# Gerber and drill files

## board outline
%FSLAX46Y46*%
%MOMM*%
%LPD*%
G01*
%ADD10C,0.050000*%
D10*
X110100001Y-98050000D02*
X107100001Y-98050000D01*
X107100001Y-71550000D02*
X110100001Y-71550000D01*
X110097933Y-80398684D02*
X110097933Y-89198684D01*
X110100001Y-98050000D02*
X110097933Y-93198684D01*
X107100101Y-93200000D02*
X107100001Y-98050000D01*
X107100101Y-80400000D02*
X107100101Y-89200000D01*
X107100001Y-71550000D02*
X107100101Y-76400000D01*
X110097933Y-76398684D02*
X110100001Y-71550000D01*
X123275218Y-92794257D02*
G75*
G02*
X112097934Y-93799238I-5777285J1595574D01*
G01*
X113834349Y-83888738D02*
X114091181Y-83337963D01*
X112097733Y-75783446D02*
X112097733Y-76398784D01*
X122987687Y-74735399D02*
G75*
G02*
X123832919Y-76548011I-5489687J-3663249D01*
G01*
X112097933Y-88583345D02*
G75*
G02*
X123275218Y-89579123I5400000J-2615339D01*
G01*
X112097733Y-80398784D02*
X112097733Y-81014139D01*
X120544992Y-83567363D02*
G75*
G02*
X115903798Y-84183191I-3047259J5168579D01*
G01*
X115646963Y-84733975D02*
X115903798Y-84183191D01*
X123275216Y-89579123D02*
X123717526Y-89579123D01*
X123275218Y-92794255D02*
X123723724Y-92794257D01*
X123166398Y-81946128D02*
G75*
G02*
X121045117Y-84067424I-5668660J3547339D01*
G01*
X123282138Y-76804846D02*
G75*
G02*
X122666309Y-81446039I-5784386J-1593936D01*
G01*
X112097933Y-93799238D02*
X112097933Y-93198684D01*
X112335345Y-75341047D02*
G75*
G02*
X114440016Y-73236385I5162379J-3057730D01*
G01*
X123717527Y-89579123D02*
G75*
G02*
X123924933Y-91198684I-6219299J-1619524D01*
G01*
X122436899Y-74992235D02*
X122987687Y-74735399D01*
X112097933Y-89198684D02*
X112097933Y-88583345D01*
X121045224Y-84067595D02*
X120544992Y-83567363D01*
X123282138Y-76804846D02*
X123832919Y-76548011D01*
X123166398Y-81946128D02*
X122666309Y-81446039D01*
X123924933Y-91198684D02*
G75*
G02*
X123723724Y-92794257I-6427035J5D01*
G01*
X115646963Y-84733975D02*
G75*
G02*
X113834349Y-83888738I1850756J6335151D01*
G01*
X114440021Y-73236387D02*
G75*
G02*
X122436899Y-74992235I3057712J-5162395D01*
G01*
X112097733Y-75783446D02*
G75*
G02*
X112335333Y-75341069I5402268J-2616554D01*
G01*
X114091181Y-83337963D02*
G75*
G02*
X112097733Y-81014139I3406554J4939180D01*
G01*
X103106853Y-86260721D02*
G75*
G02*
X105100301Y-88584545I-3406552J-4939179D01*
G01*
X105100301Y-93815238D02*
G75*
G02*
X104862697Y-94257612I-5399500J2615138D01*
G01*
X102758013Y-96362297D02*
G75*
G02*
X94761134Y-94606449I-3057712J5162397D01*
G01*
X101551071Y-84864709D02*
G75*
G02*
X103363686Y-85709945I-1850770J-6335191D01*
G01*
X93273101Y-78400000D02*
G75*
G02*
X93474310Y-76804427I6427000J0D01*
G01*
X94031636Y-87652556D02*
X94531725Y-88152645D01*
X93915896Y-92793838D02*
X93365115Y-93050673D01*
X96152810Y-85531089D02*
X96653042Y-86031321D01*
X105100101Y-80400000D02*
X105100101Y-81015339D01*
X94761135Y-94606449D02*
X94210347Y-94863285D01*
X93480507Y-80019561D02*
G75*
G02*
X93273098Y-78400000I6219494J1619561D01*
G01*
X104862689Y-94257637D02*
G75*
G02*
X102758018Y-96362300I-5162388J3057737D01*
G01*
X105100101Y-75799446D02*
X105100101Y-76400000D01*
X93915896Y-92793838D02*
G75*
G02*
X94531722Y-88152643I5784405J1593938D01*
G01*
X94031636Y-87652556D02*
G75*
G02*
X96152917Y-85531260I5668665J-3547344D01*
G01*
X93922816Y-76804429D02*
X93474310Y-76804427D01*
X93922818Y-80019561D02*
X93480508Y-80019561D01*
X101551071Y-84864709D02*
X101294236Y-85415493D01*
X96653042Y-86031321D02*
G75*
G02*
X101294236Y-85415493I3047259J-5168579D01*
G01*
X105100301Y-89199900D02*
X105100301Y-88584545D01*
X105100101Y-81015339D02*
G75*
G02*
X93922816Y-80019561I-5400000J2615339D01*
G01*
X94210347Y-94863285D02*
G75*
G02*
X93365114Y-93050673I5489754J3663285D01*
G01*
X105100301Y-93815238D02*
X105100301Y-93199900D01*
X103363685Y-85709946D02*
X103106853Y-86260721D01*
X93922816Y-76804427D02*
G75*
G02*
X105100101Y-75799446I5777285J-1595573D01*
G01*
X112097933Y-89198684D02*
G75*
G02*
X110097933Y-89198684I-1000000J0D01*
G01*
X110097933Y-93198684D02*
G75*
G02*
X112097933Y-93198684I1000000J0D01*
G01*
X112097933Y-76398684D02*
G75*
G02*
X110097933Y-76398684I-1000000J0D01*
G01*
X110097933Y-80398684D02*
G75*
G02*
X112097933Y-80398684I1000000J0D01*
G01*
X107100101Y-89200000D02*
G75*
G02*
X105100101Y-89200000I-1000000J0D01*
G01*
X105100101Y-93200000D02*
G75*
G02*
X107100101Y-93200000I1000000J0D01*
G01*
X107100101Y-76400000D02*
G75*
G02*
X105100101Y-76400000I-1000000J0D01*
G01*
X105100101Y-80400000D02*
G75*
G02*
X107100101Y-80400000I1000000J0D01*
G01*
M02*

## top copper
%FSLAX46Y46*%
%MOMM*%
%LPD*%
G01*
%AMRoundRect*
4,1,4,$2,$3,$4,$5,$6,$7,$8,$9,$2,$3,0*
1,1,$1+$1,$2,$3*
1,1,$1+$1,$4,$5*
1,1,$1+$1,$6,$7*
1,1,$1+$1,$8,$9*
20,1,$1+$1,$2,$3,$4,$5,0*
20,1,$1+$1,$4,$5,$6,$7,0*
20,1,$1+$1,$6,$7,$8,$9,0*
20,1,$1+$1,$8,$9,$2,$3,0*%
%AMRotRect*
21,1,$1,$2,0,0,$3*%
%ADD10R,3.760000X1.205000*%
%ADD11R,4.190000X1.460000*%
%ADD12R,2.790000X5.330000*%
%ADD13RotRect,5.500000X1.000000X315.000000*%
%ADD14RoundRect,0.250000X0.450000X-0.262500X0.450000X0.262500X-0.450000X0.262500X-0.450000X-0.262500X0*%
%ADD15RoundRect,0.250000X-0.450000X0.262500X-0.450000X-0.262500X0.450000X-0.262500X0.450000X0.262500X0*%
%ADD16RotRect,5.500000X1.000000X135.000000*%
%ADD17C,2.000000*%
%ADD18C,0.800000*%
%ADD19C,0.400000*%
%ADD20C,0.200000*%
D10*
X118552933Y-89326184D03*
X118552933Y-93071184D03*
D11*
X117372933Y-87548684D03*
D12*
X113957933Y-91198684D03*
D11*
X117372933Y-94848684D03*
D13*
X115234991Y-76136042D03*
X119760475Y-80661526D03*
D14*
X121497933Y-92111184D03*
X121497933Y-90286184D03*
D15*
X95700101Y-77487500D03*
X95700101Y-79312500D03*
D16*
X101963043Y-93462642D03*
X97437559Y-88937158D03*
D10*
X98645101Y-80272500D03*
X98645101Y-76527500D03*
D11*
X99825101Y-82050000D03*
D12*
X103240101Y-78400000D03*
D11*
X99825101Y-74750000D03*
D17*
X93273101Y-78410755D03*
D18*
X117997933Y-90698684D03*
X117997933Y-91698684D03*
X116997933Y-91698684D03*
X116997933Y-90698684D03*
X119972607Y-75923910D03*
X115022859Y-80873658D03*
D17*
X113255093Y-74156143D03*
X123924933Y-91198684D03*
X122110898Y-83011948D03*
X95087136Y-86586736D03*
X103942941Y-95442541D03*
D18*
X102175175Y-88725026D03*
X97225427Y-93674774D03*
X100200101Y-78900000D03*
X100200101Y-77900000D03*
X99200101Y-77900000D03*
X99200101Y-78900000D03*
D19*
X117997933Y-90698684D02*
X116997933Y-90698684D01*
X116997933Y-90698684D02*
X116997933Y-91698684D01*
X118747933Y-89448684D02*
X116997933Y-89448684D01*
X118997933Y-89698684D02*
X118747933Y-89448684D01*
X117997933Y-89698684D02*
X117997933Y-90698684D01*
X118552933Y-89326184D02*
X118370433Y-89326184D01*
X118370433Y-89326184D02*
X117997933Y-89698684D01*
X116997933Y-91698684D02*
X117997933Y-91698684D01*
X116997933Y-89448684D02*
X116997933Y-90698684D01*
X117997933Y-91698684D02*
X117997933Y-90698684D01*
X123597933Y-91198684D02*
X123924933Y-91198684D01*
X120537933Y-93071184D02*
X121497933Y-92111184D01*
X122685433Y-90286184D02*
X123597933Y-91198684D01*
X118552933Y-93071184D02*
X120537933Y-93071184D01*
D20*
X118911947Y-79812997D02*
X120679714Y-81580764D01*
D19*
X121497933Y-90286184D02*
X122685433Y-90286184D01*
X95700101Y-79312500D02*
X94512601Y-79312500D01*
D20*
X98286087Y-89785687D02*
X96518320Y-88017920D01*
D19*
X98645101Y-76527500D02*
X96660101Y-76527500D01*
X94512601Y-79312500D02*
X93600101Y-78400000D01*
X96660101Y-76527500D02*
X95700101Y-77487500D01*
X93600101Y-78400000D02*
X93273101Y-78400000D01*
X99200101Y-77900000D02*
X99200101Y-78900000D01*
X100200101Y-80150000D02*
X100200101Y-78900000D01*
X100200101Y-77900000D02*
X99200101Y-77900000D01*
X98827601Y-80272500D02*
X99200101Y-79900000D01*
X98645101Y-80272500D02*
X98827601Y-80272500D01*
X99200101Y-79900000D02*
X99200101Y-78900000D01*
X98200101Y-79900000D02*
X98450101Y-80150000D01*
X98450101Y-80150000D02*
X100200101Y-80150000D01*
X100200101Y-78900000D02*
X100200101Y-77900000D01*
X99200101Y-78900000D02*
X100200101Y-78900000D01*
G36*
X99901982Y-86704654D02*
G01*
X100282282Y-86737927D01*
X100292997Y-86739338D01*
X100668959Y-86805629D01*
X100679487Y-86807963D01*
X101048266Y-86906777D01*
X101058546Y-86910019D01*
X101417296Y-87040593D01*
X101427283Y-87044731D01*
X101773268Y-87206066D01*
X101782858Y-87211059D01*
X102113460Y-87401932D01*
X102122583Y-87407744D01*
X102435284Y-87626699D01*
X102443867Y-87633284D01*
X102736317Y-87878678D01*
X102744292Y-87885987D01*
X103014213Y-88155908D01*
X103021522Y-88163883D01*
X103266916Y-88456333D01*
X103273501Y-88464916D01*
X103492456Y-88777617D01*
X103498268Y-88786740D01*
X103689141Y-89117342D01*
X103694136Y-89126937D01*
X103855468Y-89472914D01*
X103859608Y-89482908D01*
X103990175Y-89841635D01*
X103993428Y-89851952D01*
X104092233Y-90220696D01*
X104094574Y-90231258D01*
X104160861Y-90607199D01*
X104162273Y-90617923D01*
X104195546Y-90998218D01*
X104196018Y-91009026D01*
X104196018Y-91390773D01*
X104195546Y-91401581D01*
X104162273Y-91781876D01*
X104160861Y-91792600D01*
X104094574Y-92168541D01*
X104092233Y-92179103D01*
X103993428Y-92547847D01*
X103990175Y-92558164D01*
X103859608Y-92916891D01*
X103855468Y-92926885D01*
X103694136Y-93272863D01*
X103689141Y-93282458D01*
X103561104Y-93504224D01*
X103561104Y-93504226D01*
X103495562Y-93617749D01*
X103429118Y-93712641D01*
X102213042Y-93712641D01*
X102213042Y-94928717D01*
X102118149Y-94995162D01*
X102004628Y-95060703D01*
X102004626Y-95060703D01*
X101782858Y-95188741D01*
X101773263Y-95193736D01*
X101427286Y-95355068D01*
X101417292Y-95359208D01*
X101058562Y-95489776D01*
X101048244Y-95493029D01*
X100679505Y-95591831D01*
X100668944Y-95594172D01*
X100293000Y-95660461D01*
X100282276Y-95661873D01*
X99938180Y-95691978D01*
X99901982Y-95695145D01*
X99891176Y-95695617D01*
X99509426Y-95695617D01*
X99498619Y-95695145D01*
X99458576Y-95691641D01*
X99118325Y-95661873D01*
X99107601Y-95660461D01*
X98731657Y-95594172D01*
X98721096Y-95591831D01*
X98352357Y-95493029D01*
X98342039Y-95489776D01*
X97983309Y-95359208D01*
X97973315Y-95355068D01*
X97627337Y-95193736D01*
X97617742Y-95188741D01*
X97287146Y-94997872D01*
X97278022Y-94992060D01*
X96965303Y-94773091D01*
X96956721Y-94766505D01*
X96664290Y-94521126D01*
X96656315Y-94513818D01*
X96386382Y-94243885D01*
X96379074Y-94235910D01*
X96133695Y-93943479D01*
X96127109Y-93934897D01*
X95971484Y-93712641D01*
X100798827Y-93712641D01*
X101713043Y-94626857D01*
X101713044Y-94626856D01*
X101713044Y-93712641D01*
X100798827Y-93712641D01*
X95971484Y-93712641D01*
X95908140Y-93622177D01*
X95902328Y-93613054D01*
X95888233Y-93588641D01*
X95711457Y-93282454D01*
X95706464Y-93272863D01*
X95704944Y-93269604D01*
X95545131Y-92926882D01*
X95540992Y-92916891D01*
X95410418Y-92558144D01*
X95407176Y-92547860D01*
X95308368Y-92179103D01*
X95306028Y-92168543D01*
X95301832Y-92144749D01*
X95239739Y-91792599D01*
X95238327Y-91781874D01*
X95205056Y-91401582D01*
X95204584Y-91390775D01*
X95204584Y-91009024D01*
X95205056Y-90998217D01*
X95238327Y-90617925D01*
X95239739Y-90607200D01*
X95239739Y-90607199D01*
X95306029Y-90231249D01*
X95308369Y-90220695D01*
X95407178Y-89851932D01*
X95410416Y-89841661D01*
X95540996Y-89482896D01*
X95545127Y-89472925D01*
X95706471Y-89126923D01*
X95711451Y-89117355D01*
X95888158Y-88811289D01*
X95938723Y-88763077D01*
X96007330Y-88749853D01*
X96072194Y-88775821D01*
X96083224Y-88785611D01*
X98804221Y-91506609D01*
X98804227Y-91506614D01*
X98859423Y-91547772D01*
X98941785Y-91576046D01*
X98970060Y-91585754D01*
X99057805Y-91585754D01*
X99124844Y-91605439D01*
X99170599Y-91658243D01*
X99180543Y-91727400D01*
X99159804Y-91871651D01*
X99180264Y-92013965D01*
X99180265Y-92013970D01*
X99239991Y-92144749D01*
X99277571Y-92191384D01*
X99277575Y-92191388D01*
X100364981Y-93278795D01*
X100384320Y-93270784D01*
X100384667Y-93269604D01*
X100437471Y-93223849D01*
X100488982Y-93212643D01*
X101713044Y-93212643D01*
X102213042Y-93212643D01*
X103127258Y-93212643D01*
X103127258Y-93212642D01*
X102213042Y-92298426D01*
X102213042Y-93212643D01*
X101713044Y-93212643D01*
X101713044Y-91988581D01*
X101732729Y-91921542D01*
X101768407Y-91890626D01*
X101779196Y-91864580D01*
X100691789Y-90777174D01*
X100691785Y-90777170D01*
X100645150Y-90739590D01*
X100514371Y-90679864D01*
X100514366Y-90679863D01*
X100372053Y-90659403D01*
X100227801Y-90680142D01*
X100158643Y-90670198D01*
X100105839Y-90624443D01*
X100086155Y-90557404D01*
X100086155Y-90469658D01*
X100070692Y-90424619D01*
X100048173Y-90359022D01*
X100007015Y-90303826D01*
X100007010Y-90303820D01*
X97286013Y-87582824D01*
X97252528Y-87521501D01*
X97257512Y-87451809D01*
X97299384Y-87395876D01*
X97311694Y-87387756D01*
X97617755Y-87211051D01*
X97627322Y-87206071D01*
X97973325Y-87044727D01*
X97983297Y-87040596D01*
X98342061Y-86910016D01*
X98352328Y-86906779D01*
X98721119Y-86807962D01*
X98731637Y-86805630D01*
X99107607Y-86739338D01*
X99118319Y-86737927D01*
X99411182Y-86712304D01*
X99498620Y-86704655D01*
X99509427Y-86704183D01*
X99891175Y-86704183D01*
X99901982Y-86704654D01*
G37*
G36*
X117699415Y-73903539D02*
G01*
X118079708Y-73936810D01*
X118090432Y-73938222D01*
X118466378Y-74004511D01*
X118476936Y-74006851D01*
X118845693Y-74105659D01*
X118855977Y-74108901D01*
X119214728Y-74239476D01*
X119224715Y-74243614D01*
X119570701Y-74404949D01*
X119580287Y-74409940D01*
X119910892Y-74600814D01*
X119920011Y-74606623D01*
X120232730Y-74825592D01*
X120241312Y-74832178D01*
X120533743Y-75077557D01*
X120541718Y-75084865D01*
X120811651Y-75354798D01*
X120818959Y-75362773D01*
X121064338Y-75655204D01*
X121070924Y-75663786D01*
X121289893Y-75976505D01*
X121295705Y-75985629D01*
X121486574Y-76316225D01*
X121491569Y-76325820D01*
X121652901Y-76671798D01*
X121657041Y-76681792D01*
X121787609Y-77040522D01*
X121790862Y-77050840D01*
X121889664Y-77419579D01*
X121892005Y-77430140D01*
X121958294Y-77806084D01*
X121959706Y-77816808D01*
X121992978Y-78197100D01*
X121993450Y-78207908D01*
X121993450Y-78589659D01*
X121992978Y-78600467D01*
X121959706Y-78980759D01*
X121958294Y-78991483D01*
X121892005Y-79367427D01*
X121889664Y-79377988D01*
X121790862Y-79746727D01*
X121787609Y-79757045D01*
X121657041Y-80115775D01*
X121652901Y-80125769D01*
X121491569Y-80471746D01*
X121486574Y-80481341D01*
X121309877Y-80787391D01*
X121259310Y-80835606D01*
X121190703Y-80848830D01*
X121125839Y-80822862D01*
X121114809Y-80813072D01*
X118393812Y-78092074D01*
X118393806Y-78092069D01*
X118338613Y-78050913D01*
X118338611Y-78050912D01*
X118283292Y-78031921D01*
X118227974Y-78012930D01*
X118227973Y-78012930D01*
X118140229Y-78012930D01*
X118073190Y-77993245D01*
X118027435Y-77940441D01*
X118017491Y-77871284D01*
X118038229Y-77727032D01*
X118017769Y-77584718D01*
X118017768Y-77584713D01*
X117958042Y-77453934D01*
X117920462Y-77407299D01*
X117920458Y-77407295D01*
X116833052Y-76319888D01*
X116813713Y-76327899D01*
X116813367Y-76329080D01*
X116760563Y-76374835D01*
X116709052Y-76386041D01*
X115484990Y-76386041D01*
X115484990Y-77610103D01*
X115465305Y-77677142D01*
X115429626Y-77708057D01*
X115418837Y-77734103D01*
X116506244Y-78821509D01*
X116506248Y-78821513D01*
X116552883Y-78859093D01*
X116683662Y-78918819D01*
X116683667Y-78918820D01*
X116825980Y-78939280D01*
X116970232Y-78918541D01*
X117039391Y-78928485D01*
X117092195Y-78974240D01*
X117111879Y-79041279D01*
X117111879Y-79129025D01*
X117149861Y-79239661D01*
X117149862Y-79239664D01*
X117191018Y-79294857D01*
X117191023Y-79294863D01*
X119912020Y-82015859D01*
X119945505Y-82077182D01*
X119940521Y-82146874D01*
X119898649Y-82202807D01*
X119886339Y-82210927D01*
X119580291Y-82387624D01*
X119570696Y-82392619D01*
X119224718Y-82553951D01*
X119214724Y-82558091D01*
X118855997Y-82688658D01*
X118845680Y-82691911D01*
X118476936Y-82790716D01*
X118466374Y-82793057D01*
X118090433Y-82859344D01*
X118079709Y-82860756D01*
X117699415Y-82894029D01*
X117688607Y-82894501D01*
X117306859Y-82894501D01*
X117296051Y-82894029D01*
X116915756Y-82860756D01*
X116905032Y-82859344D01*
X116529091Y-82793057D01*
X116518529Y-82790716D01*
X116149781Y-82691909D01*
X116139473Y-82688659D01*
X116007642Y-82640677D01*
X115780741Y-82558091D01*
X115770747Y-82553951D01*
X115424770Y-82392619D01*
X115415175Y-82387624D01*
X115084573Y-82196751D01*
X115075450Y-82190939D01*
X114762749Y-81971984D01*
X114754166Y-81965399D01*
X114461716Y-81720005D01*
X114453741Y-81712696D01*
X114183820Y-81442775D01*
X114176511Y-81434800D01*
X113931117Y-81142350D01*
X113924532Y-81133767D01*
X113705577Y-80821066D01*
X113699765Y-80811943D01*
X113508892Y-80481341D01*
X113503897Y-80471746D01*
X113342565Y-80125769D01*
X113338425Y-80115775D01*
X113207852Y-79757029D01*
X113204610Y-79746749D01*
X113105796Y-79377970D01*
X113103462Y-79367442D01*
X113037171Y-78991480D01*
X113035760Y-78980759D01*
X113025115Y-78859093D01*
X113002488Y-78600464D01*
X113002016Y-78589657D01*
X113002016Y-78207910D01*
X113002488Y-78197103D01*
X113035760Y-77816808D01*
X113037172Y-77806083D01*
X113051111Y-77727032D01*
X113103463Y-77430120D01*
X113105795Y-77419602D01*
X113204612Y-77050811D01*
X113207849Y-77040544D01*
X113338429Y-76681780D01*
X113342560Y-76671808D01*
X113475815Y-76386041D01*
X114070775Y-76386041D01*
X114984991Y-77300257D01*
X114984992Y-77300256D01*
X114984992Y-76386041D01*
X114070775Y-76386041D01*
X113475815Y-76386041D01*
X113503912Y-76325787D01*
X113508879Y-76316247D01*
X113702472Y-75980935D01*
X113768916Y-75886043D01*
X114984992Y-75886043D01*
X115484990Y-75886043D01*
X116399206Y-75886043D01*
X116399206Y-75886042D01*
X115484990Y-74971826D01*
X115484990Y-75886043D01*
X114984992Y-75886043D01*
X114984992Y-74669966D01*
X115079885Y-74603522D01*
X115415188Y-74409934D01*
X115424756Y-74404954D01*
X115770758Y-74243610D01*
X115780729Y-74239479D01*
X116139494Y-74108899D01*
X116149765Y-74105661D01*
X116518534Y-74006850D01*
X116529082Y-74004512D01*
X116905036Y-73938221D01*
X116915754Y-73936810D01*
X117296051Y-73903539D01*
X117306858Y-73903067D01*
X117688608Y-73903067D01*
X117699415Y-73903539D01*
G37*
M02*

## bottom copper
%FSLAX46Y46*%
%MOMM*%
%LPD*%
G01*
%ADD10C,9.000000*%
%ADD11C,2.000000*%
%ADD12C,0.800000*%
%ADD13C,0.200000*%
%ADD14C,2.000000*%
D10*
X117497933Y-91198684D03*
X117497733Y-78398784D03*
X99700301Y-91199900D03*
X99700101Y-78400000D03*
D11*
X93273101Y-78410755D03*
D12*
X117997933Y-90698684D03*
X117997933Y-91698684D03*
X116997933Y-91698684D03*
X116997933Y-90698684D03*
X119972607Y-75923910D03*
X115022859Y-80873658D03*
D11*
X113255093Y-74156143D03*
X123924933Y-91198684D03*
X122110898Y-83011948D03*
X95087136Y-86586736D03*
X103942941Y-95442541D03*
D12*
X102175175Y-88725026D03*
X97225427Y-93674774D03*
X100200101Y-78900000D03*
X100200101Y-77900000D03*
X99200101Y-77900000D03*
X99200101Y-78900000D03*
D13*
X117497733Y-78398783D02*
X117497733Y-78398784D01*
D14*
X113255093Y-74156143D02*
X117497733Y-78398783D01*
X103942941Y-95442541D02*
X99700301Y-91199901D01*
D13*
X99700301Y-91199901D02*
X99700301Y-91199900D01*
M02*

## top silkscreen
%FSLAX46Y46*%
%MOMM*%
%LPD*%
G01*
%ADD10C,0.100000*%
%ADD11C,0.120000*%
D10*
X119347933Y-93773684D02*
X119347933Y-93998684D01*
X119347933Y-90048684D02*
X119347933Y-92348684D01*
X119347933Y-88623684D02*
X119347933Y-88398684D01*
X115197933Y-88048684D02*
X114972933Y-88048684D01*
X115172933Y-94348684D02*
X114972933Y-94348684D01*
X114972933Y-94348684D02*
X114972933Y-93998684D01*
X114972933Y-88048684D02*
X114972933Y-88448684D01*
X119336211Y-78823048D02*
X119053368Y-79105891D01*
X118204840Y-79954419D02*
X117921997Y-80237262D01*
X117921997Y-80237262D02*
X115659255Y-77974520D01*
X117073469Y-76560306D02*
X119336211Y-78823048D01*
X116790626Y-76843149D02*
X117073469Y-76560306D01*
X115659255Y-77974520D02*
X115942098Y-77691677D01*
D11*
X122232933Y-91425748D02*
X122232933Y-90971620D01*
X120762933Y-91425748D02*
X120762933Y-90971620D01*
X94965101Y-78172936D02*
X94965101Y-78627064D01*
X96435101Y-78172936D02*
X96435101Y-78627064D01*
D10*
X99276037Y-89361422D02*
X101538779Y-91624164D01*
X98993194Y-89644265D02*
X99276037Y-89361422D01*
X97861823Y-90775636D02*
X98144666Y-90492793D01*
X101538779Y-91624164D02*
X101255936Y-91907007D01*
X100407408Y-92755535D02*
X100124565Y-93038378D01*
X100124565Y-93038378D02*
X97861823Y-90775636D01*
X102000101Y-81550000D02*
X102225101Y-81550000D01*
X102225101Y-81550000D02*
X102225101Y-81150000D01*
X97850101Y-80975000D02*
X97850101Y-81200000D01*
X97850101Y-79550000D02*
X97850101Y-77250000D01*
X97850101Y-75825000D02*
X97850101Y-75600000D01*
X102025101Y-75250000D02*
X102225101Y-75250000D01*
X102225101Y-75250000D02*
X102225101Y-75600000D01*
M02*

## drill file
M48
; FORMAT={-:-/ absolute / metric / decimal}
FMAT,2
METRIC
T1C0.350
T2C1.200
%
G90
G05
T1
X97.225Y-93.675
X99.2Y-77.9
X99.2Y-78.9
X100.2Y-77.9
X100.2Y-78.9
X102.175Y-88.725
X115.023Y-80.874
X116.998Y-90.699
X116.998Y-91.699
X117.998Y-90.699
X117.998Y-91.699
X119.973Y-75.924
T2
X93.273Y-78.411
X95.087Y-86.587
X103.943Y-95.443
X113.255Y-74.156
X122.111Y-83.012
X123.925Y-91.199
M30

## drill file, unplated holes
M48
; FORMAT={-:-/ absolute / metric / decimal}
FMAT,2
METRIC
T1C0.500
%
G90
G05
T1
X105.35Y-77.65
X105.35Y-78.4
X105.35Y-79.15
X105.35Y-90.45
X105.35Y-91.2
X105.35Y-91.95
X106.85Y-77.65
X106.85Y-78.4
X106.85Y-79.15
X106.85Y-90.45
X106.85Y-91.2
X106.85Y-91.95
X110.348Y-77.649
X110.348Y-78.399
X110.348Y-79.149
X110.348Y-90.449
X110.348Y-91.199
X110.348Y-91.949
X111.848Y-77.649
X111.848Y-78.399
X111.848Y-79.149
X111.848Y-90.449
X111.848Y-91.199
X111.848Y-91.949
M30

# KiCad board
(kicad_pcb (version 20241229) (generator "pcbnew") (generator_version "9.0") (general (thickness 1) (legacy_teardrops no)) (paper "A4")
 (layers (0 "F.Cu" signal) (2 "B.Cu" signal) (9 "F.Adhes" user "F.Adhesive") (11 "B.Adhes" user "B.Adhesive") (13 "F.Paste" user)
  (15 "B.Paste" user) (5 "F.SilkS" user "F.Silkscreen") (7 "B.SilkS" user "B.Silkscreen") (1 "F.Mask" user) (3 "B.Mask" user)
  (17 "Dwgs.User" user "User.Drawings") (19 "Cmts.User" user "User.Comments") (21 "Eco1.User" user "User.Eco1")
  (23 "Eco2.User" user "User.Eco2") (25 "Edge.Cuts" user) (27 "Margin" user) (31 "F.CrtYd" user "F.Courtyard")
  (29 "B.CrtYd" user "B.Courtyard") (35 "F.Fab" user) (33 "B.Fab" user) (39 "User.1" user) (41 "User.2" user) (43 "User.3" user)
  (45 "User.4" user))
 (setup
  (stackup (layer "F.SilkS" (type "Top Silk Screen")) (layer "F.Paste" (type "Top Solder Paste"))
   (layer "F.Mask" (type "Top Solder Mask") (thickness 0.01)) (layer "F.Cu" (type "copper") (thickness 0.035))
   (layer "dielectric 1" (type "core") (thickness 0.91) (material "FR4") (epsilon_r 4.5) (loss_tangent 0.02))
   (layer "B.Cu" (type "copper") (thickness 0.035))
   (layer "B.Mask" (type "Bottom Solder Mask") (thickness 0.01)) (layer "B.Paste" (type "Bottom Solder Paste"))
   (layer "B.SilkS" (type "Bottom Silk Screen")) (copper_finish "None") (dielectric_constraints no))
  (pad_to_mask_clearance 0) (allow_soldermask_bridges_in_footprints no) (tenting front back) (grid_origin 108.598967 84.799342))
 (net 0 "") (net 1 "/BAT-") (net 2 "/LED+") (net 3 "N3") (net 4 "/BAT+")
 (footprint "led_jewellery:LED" (layer "F.Cu") (at 99.700301 91.1999 135)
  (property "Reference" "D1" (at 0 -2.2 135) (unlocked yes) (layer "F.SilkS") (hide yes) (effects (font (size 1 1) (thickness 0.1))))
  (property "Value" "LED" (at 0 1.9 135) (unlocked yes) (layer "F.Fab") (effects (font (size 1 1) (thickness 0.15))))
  (fp_line (start 1.6 -1) (end 1.6 -0.6) (stroke (width 0.1) (type default)) (layer "F.SilkS"))
  (fp_line (start 1.6 0.6) (end 1.6 1) (stroke (width 0.1) (type default)) (layer "F.SilkS"))
  (fp_line (start 1.6 1) (end -1.6 1) (stroke (width 0.1) (type default)) (layer "F.SilkS"))
  (fp_line (start -1.6 -1) (end 1.6 -1) (stroke (width 0.1) (type default)) (layer "F.SilkS"))
  (fp_line (start -1.6 -0.6) (end -1.6 -1) (stroke (width 0.1) (type default)) (layer "F.SilkS"))
  (fp_line (start -1.6 1) (end -1.6 0.6) (stroke (width 0.1) (type default)) (layer "F.SilkS"))
  (pad "1" smd rect (at -3.2 0 135) (size 5.5 1) (layers "F.Cu" "F.Mask") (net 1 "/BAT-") (thermal_bridge_angle 45))
  (pad "2" smd rect (at 3.2 0 135) (size 5.5 1) (layers "F.Cu" "F.Mask") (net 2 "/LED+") (thermal_bridge_angle 45)))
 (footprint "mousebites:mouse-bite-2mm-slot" (layer "F.Cu") (at 106.100101 78.4 90)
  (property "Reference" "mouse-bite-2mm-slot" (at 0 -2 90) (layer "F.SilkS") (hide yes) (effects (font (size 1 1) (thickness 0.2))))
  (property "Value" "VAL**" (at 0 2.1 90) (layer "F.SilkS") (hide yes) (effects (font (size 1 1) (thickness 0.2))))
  (fp_arc (start -2 -1) (mid -1 0) (end -2 1) (stroke (width 0.05) (type solid)) (layer "Edge.Cuts"))
  (fp_arc (start 2 1) (mid 1 0) (end 2 -1) (stroke (width 0.05) (type solid)) (layer "Edge.Cuts"))
  (pad "" np_thru_hole circle (at -0.75 -0.75 90) (size 0.5 0.5) (drill 0.5) (layers "*.Cu" "*.Mask"))
  (pad "" np_thru_hole circle (at -0.75 0.75 90) (size 0.5 0.5) (drill 0.5) (layers "*.Cu" "*.Mask"))
  (pad "" np_thru_hole circle (at 0 -0.75 90) (size 0.5 0.5) (drill 0.5) (layers "*.Cu" "*.Mask"))
  (pad "" np_thru_hole circle (at 0 0.75 90) (size 0.5 0.5) (drill 0.5) (layers "*.Cu" "*.Mask"))
  (pad "" np_thru_hole circle (at 0.75 -0.75 90) (size 0.5 0.5) (drill 0.5) (layers "*.Cu" "*.Mask"))
  (pad "" np_thru_hole circle (at 0.75 0.75 90) (size 0.5 0.5) (drill 0.5) (layers "*.Cu" "*.Mask")))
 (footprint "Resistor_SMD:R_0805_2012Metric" (layer "F.Cu") (at 95.700101 78.4 -90)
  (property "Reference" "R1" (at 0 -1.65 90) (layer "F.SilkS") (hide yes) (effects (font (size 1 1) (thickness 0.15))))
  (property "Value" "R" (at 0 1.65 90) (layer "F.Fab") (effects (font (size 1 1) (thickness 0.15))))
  (fp_line (start -0.227064 0.735) (end 0.227064 0.735) (stroke (width 0.12) (type solid)) (layer "F.SilkS"))
  (fp_line (start -0.227064 -0.735) (end 0.227064 -0.735) (stroke (width 0.12) (type solid)) (layer "F.SilkS"))
  (pad "1" smd roundrect (at -0.9125 0 270) (size 1.025 1.4) (layers "F.Cu" "F.Mask" "F.Paste") (roundrect_rratio 0.243902) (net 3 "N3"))
  (pad "2" smd roundrect (at 0.9125 0 270) (size 1.025 1.4) (layers "F.Cu" "F.Mask" "F.Paste") (roundrect_rratio 0.243902) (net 2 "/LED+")))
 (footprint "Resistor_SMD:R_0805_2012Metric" (layer "F.Cu") (at 121.497933 91.198684 90)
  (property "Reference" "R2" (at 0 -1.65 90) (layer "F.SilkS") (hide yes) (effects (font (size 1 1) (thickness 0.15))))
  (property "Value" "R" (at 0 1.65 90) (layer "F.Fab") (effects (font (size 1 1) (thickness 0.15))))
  (fp_line (start -0.227064 -0.735) (end 0.227064 -0.735) (stroke (width 0.12) (type solid)) (layer "F.SilkS"))
  (fp_line (start -0.227064 0.735) (end 0.227064 0.735) (stroke (width 0.12) (type solid)) (layer "F.SilkS"))
  (pad "1" smd roundrect (at -0.9125 0 90) (size 1.025 1.4) (layers "F.Cu" "F.Mask" "F.Paste") (roundrect_rratio 0.243902) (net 3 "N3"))
  (pad "2" smd roundrect (at 0.9125 0 90) (size 1.025 1.4) (layers "F.Cu" "F.Mask" "F.Paste") (roundrect_rratio 0.243902) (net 2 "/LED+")))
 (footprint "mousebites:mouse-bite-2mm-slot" (layer "F.Cu") (at 111.097933 78.398684 -90)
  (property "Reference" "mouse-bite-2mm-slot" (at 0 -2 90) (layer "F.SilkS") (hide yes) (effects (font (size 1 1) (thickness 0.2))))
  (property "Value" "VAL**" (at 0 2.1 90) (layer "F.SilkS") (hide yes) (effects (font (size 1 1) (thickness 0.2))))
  (fp_arc (start 2 1) (mid 1 0) (end 2 -1) (stroke (width 0.05) (type solid)) (layer "Edge.Cuts"))
  (fp_arc (start -2 -1) (mid -1 0) (end -2 1) (stroke (width 0.05) (type solid)) (layer "Edge.Cuts"))
  (pad "" np_thru_hole circle (at -0.75 -0.75 270) (size 0.5 0.5) (drill 0.5) (layers "*.Cu" "*.Mask"))
  (pad "" np_thru_hole circle (at -0.75 0.75 270) (size 0.5 0.5) (drill 0.5) (layers "*.Cu" "*.Mask"))
  (pad "" np_thru_hole circle (at 0 -0.75 270) (size 0.5 0.5) (drill 0.5) (layers "*.Cu" "*.Mask"))
  (pad "" np_thru_hole circle (at 0 0.75 270) (size 0.5 0.5) (drill 0.5) (layers "*.Cu" "*.Mask"))
  (pad "" np_thru_hole circle (at 0.75 -0.75 270) (size 0.5 0.5) (drill 0.5) (layers "*.Cu" "*.Mask"))
  (pad "" np_thru_hole circle (at 0.75 0.75 270) (size 0.5 0.5) (drill 0.5) (layers "*.Cu" "*.Mask")))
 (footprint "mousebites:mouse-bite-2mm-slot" (layer "F.Cu") (at 111.097933 91.198684 -90)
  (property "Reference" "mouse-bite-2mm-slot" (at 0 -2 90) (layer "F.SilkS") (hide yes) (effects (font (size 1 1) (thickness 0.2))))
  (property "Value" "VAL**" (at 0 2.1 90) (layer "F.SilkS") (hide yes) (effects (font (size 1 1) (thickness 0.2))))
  (fp_arc (start 2 1) (mid 1 0) (end 2 -1) (stroke (width 0.05) (type solid)) (layer "Edge.Cuts"))
  (fp_arc (start -2 -1) (mid -1 0) (end -2 1) (stroke (width 0.05) (type solid)) (layer "Edge.Cuts"))
  (pad "" np_thru_hole circle (at -0.75 -0.75 270) (size 0.5 0.5) (drill 0.5) (layers "*.Cu" "*.Mask"))
  (pad "" np_thru_hole circle (at -0.75 0.75 270) (size 0.5 0.5) (drill 0.5) (layers "*.Cu" "*.Mask"))
  (pad "" np_thru_hole circle (at 0 -0.75 270) (size 0.5 0.5) (drill 0.5) (layers "*.Cu" "*.Mask"))
  (pad "" np_thru_hole circle (at 0 0.75 270) (size 0.5 0.5) (drill 0.5) (layers "*.Cu" "*.Mask"))
  (pad "" np_thru_hole circle (at 0.75 -0.75 270) (size 0.5 0.5) (drill 0.5) (layers "*.Cu" "*.Mask"))
  (pad "" np_thru_hole circle (at 0.75 0.75 270) (size 0.5 0.5) (drill 0.5) (layers "*.Cu" "*.Mask")))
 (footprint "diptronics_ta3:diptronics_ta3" (layer "F.Cu") (at 102.225101 78.4 90)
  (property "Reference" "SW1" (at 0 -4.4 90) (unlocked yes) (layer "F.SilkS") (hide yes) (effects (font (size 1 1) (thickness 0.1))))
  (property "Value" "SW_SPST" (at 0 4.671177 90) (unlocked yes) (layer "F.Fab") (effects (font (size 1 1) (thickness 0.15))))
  (fp_line (start 2.575 -4.375) (end 2.8 -4.375) (stroke (width 0.1) (type default)) (layer "F.SilkS"))
  (fp_line (start -1.15 -4.375) (end 1.15 -4.375) (stroke (width 0.1) (type default)) (layer "F.SilkS"))
  (fp_line (start -2.575 -4.375) (end -2.8 -4.375) (stroke (width 0.1) (type default)) (layer "F.SilkS"))
  (fp_line (start -3.15 -0.225) (end -3.15 0) (stroke (width 0.1) (type default)) (layer "F.SilkS"))
  (fp_line (start 3.15 -0.2) (end 3.15 0) (stroke (width 0.1) (type default)) (layer "F.SilkS"))
  (fp_line (start 3.15 0) (end 2.8 0) (stroke (width 0.1) (type default)) (layer "F.SilkS"))
  (fp_line (start -3.15 0) (end -2.75 0) (stroke (width 0.1) (type default)) (layer "F.SilkS"))
  (pad "1" smd rect (at -1.8725 -3.58 180) (size 3.76 1.205) (layers "F.Cu" "F.Mask" "F.Paste") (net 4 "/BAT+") (thermal_bridge_angle 45))
  (pad "2" smd rect (at 1.8725 -3.58 180) (size 3.76 1.205) (layers "F.Cu" "F.Mask" "F.Paste") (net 3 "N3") (thermal_bridge_angle 45))
  (pad "MP" smd rect (at -3.65 -2.4 90) (size 1.46 4.19) (layers "F.Cu" "F.Mask" "F.Paste") (thermal_bridge_angle 45))
  (pad "MP" smd rect (at 0 1.015 90) (size 5.33 2.79) (layers "F.Cu" "F.Mask" "F.Paste") (thermal_bridge_angle 45))
  (pad "MP" smd rect (at 3.65 -2.4 90) (size 1.46 4.19) (layers "F.Cu" "F.Mask" "F.Paste") (thermal_bridge_angle 45)))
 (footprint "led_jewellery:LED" (layer "F.Cu") (at 117.497733 78.398784 -45)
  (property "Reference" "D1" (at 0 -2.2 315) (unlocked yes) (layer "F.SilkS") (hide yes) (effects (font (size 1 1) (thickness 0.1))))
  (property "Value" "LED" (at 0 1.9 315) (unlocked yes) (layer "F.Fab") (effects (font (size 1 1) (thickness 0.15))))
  (fp_line (start -1.6 1) (end -1.6 0.6) (stroke (width 0.1) (type default)) (layer "F.SilkS"))
  (fp_line (start -1.6 -0.6) (end -1.6 -1) (stroke (width 0.1) (type default)) (layer "F.SilkS"))
  (fp_line (start -1.6 -1) (end 1.6 -1) (stroke (width 0.1) (type default)) (layer "F.SilkS"))
  (fp_line (start 1.6 1) (end -1.6 1) (stroke (width 0.1) (type default)) (layer "F.SilkS"))
  (fp_line (start 1.6 0.6) (end 1.6 1) (stroke (width 0.1) (type default)) (layer "F.SilkS"))
  (fp_line (start 1.6 -1) (end 1.6 -0.6) (stroke (width 0.1) (type default)) (layer "F.SilkS"))
  (pad "1" smd rect (at -3.2 0 315) (size 5.5 1) (layers "F.Cu" "F.Mask") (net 1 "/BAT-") (thermal_bridge_angle 45))
  (pad "2" smd rect (at 3.2 0 315) (size 5.5 1) (layers "F.Cu" "F.Mask") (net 2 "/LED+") (thermal_bridge_angle 45)))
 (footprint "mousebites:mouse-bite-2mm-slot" (layer "F.Cu") (at 106.100101 91.2 90)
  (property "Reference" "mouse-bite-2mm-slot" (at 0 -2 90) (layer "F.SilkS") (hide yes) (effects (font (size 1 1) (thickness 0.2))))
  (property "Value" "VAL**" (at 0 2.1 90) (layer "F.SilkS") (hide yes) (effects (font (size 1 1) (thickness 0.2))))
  (fp_arc (start -2 -1) (mid -1 0) (end -2 1) (stroke (width 0.05) (type solid)) (layer "Edge.Cuts"))
  (fp_arc (start 2 1) (mid 1 0) (end 2 -1) (stroke (width 0.05) (type solid)) (layer "Edge.Cuts"))
  (pad "" np_thru_hole circle (at -0.75 -0.75 90) (size 0.5 0.5) (drill 0.5) (layers "*.Cu" "*.Mask"))
  (pad "" np_thru_hole circle (at -0.75 0.75 90) (size 0.5 0.5) (drill 0.5) (layers "*.Cu" "*.Mask"))
  (pad "" np_thru_hole circle (at 0 -0.75 90) (size 0.5 0.5) (drill 0.5) (layers "*.Cu" "*.Mask"))
  (pad "" np_thru_hole circle (at 0 0.75 90) (size 0.5 0.5) (drill 0.5) (layers "*.Cu" "*.Mask"))
  (pad "" np_thru_hole circle (at 0.75 -0.75 90) (size 0.5 0.5) (drill 0.5) (layers "*.Cu" "*.Mask"))
  (pad "" np_thru_hole circle (at 0.75 0.75 90) (size 0.5 0.5) (drill 0.5) (layers "*.Cu" "*.Mask")))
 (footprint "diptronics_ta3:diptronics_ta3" (layer "F.Cu") (at 114.972933 91.198684 -90)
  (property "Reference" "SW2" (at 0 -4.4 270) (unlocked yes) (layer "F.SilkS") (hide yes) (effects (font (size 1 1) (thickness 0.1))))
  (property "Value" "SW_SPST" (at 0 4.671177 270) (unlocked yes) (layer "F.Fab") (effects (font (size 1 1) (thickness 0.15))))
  (fp_line (start -3.15 0) (end -2.75 0) (stroke (width 0.1) (type default)) (layer "F.SilkS"))
  (fp_line (start 3.15 0) (end 2.8 0) (stroke (width 0.1) (type default)) (layer "F.SilkS"))
  (fp_line (start 3.15 -0.2) (end 3.15 0) (stroke (width 0.1) (type default)) (layer "F.SilkS"))
  (fp_line (start -3.15 -0.225) (end -3.15 0) (stroke (width 0.1) (type default)) (layer "F.SilkS"))
  (fp_line (start -2.575 -4.375) (end -2.8 -4.375) (stroke (width 0.1) (type default)) (layer "F.SilkS"))
  (fp_line (start -1.15 -4.375) (end 1.15 -4.375) (stroke (width 0.1) (type default)) (layer "F.SilkS"))
  (fp_line (start 2.575 -4.375) (end 2.8 -4.375) (stroke (width 0.1) (type default)) (layer "F.SilkS"))
  (pad "1" smd rect (at -1.8725 -3.58) (size 3.76 1.205) (layers "F.Cu" "F.Mask" "F.Paste") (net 4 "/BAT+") (thermal_bridge_angle 45))
  (pad "2" smd rect (at 1.8725 -3.58) (size 3.76 1.205) (layers "F.Cu" "F.Mask" "F.Paste") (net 3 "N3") (thermal_bridge_angle 45))
  (pad "MP" smd rect (at -3.65 -2.4 270) (size 1.46 4.19) (layers "F.Cu" "F.Mask" "F.Paste") (thermal_bridge_angle 45))
  (pad "MP" smd rect (at 0 1.015 270) (size 5.33 2.79) (layers "F.Cu" "F.Mask" "F.Paste") (thermal_bridge_angle 45))
  (pad "MP" smd rect (at 3.65 -2.4 270) (size 1.46 4.19) (layers "F.Cu" "F.Mask" "F.Paste") (thermal_bridge_angle 45)))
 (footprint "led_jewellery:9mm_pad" (layer "B.Cu") (at 117.497933 91.198684 90)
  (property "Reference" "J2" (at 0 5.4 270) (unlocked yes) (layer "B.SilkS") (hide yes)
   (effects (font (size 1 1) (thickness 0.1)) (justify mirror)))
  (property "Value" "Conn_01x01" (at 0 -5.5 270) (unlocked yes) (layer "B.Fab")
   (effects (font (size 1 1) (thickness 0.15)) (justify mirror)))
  (pad "1" smd circle (at 0 0 90) (size 9 9) (layers "B.Cu" "B.Mask") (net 4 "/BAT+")))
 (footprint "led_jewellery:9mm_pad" (layer "B.Cu") (at 99.700301 91.1999 135)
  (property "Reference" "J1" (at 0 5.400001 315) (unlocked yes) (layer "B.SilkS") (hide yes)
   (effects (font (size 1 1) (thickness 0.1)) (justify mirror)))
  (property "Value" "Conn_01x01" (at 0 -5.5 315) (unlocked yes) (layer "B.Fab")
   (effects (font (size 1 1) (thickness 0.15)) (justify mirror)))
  (pad "1" smd circle (at 0 0 135) (size 9 9) (layers "B.Cu" "B.Mask") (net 1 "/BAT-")))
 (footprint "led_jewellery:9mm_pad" (layer "B.Cu") (at 117.497733 78.398784 -45)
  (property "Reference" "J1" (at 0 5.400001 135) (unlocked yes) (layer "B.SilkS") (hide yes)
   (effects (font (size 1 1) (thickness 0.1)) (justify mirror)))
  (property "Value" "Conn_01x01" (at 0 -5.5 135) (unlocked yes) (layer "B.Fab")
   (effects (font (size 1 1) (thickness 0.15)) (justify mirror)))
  (pad "1" smd circle (at 0 0 315) (size 9 9) (layers "B.Cu" "B.Mask") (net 1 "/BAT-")))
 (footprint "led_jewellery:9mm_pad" (layer "B.Cu") (at 99.700101 78.4 -90)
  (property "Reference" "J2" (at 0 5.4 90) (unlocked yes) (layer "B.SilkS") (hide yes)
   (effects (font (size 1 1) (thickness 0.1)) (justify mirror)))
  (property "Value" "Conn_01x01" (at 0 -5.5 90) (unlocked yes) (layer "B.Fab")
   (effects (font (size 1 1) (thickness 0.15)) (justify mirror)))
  (pad "1" smd circle (at 0 0 270) (size 9 9) (layers "B.Cu" "B.Mask") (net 4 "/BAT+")))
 (gr_arc (start 103.106853 86.260721) (mid 104.254297 87.293341) (end 105.100301 88.584545) (stroke (width 0.05) (type default))
  (layer "Edge.Cuts"))
 (gr_line (start 122.436899 74.992235) (end 122.987687 74.735399) (stroke (width 0.05) (type solid)) (layer "Edge.Cuts"))
 (gr_arc (start 123.166398 81.946128) (mid 122.226249 83.127267) (end 121.045117 84.067424) (stroke (width 0.05) (type default))
  (layer "Edge.Cuts"))
 (gr_line (start 123.275216 89.579123) (end 123.717526 89.579123) (stroke (width 0.05) (type default)) (layer "Edge.Cuts"))
 (gr_arc (start 105.100301 93.815238) (mid 104.986129 94.038912) (end 104.862701 94.257615) (stroke (width 0.05) (type default))
  (layer "Edge.Cuts"))
 (gr_line (start 107.100101 93.2) (end 107.100001 98.05) (stroke (width 0.05) (type default)) (layer "Edge.Cuts"))
 (gr_arc (start 102.758013 96.362297) (mid 98.413554 97.060295) (end 94.761135 94.606449) (stroke (width 0.05) (type default))
  (layer "Edge.Cuts"))
 (gr_arc (start 122.987687 74.735399) (mid 123.479364 75.609501) (end 123.832919 76.548011) (stroke (width 0.05) (type default))
  (layer "Edge.Cuts"))
 (gr_arc (start 101.551071 84.864709) (mid 102.489581 85.218269) (end 103.363685 85.709946) (stroke (width 0.05) (type default))
  (layer "Edge.Cuts"))
 (gr_line (start 112.097933 89.198684) (end 112.097933 88.583345) (stroke (width 0.05) (type default)) (layer "Edge.Cuts"))
 (gr_arc (start 93.273101 78.4) (mid 93.323602 77.595895) (end 93.47431 76.804427) (stroke (width 0.05) (type default)) (layer "Edge.Cuts"))
 (gr_line (start 112.097733 75.783446) (end 112.097733 76.398784) (stroke (width 0.05) (type default)) (layer "Edge.Cuts"))
 (gr_line (start 94.031636 87.652556) (end 94.531725 88.152645) (stroke (width 0.05) (type default)) (layer "Edge.Cuts"))
 (gr_line (start 107.100001 71.55) (end 107.100101 76.4) (stroke (width 0.05) (type default)) (layer "Edge.Cuts"))
 (gr_line (start 93.915896 92.793838) (end 93.365115 93.050673) (stroke (width 0.05) (type solid)) (layer "Edge.Cuts"))
 (gr_line (start 96.15281 85.531089) (end 96.653042 86.031321) (stroke (width 0.05) (type default)) (layer "Edge.Cuts"))
 (gr_line (start 110.097933 80.398684) (end 110.097933 89.198684) (stroke (width 0.05) (type default)) (layer "Edge.Cuts"))
 (gr_line (start 110.100001 98.05) (end 107.100001 98.05) (stroke (width 0.05) (type default)) (layer "Edge.Cuts"))
 (gr_line (start 105.100101 80.4) (end 105.100101 81.015339) (stroke (width 0.05) (type default)) (layer "Edge.Cuts"))
 (gr_arc (start 123.717527 89.579123) (mid 123.872873 90.38229) (end 123.924933 91.198684) (stroke (width 0.05) (type default))
  (layer "Edge.Cuts"))
 (gr_line (start 94.761135 94.606449) (end 94.210347 94.863285) (stroke (width 0.05) (type solid)) (layer "Edge.Cuts"))
 (gr_line (start 112.097733 80.398784) (end 112.097733 81.014139) (stroke (width 0.05) (type default)) (layer "Edge.Cuts"))
 (gr_arc (start 93.480507 80.019561) (mid 93.325161 79.216394) (end 93.273101 78.4) (stroke (width 0.05) (type default)) (layer "Edge.Cuts"))
 (gr_arc (start 123.282138 76.804846) (mid 123.445601 79.187989) (end 122.666309 81.446039) (stroke (width 0.05) (type default))
  (layer "Edge.Cuts"))
 (gr_arc (start 104.862689 94.257637) (mid 103.942934 95.442549) (end 102.758018 96.362299) (stroke (width 0.05) (type default))
  (layer "Edge.Cuts"))
 (gr_line (start 105.100101 75.799446) (end 105.100101 76.4) (stroke (width 0.05) (type default)) (layer "Edge.Cuts"))
 (gr_line (start 123.166398 81.946128) (end 122.666309 81.446039) (stroke (width 0.05) (type default)) (layer "Edge.Cuts"))
 (gr_line (start 123.275218 92.794255) (end 123.723724 92.794257) (stroke (width 0.05) (type default)) (layer "Edge.Cuts"))
 (gr_arc (start 93.915896 92.793838) (mid 93.752433 90.410695) (end 94.531725 88.152645) (stroke (width 0.05) (type default))
  (layer "Edge.Cuts"))
 (gr_arc (start 94.031636 87.652556) (mid 94.971785 86.471417) (end 96.152917 85.53126) (stroke (width 0.05) (type default))
  (layer "Edge.Cuts"))
 (gr_arc (start 112.097733 75.783446) (mid 112.211905 75.559772) (end 112.335333 75.341069) (stroke (width 0.05) (type default))
  (layer "Edge.Cuts"))
 (gr_arc (start 115.646963 84.733975) (mid 114.708453 84.380415) (end 113.834349 83.888738) (stroke (width 0.05) (type default))
  (layer "Edge.Cuts"))
 (gr_arc (start 120.544992 83.567363) (mid 118.286941 84.346653) (end 115.903798 84.183191) (stroke (width 0.05) (type default))
  (layer "Edge.Cuts"))
 (gr_line (start 93.922816 76.804429) (end 93.47431 76.804427) (stroke (width 0.05) (type default)) (layer "Edge.Cuts"))
 (gr_arc (start 123.924933 91.198684) (mid 123.874432 92.002789) (end 123.723724 92.794257) (stroke (width 0.05) (type default))
  (layer "Edge.Cuts"))
 (gr_line (start 112.097933 93.799238) (end 112.097933 93.198684) (stroke (width 0.05) (type default)) (layer "Edge.Cuts"))
 (gr_arc (start 123.275218 92.794257) (mid 118.034666 97.168172) (end 112.097933 93.799238) (stroke (width 0.05) (type default))
  (layer "Edge.Cuts"))
 (gr_line (start 123.282138 76.804846) (end 123.832919 76.548011) (stroke (width 0.05) (type solid)) (layer "Edge.Cuts"))
 (gr_line (start 93.922818 80.019561) (end 93.480508 80.019561) (stroke (width 0.05) (type default)) (layer "Edge.Cuts"))
 (gr_line (start 121.045224 84.067595) (end 120.544992 83.567363) (stroke (width 0.05) (type default)) (layer "Edge.Cuts"))
 (gr_line (start 101.551071 84.864709) (end 101.294236 85.415493) (stroke (width 0.05) (type solid)) (layer "Edge.Cuts"))
 (gr_line (start 107.100101 80.4) (end 107.100101 89.2) (stroke (width 0.05) (type default)) (layer "Edge.Cuts"))
 (gr_arc (start 114.440021 73.236387) (mid 118.78448 72.538389) (end 122.436899 74.992235) (stroke (width 0.05) (type default))
  (layer "Edge.Cuts"))
 (gr_arc (start 96.653042 86.031321) (mid 98.911093 85.252031) (end 101.294236 85.415493) (stroke (width 0.05) (type default))
  (layer "Edge.Cuts"))
 (gr_line (start 105.100301 89.1999) (end 105.100301 88.584545) (stroke (width 0.05) (type default)) (layer "Edge.Cuts"))
 (gr_arc (start 105.100101 81.015339) (mid 99.167673 84.37633) (end 93.922816 80.019561) (stroke (width 0.05) (type default))
  (layer "Edge.Cuts"))
 (gr_arc (start 94.210347 94.863285) (mid 93.71867 93.989183) (end 93.365115 93.050673) (stroke (width 0.05) (type default))
  (layer "Edge.Cuts"))
 (gr_line (start 110.097933 76.398684) (end 110.100001 71.55) (stroke (width 0.05) (type default)) (layer "Edge.Cuts"))
 (gr_line (start 107.100001 71.55) (end 110.100001 71.55) (stroke (width 0.05) (type default)) (layer "Edge.Cuts"))
 (gr_line (start 105.100301 93.815238) (end 105.100301 93.1999) (stroke (width 0.05) (type default)) (layer "Edge.Cuts"))
 (gr_arc (start 112.335345 75.341047) (mid 113.2551 74.156135) (end 114.440016 73.236385) (stroke (width 0.05) (type default))
  (layer "Edge.Cuts"))
 (gr_line (start 110.100001 98.05) (end 110.097933 93.198684) (stroke (width 0.05) (type default)) (layer "Edge.Cuts"))
 (gr_arc (start 112.097933 88.583345) (mid 118.030361 85.222354) (end 123.275218 89.579123) (stroke (width 0.05) (type default))
  (layer "Edge.Cuts"))
 (gr_arc (start 114.091181 83.337963) (mid 112.943737 82.305343) (end 112.097733 81.014139) (stroke (width 0.05) (type default))
  (layer "Edge.Cuts"))
 (gr_line (start 103.363685 85.709946) (end 103.106853 86.260721) (stroke (width 0.05) (type solid)) (layer "Edge.Cuts"))
 (gr_line (start 113.834349 83.888738) (end 114.091181 83.337963) (stroke (width 0.05) (type solid)) (layer "Edge.Cuts"))
 (gr_line (start 115.646963 84.733975) (end 115.903798 84.183191) (stroke (width 0.05) (type solid)) (layer "Edge.Cuts"))
 (gr_arc (start 93.922816 76.804427) (mid 99.163368 72.430512) (end 105.100101 75.799446) (stroke (width 0.05) (type default))
  (layer "Edge.Cuts"))
 (segment (start 98.645101 76.5275) (end 96.660101 76.5275) (width 0.4) (layer "F.Cu") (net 3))
 (segment (start 118.552933 93.071184) (end 120.537933 93.071184) (width 0.4) (layer "F.Cu") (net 3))
 (segment (start 120.537933 93.071184) (end 121.497933 92.111184) (width 0.4) (layer "F.Cu") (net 3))
 (segment (start 96.660101 76.5275) (end 95.700101 77.4875) (width 0.4) (layer "F.Cu") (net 3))
 (segment (start 98.286087 89.785687) (end 96.51832 88.01792) (width 0.2) (layer "F.Cu") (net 2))
 (segment (start 122.685433 90.286184) (end 123.597933 91.198684) (width 0.4) (layer "F.Cu") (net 2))
 (segment (start 123.597933 91.198684) (end 123.924933 91.198684) (width 0.4) (layer "F.Cu") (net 2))
 (segment (start 118.911947 79.812997) (end 120.679714 81.580764) (width 0.2) (layer "F.Cu") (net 2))
 (segment (start 121.497933 90.286184) (end 122.685433 90.286184) (width 0.4) (layer "F.Cu") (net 2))
 (segment (start 94.512601 79.3125) (end 93.600101 78.4) (width 0.4) (layer "F.Cu") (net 2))
 (segment (start 95.700101 79.3125) (end 94.512601 79.3125) (width 0.4) (layer "F.Cu") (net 2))
 (segment (start 93.600101 78.4) (end 93.273101 78.4) (width 0.4) (layer "F.Cu") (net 2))
 (via (at 95.087136 86.586736) (size 2) (drill 1.2) (layers "F.Cu" "B.Cu") (free yes) (tenting none) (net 2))
 (via (at 93.273101 78.410755) (size 2) (drill 1.2) (layers "F.Cu" "B.Cu") (free yes) (tenting none) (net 2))
 (via (at 122.110898 83.011948) (size 2) (drill 1.2) (layers "F.Cu" "B.Cu") (free yes) (tenting none) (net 2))
 (via (at 123.924933 91.198684) (size 2) (drill 1.2) (layers "F.Cu" "B.Cu") (free yes) (tenting none) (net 2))
 (via (at 102.175175 88.725026) (size 0.8) (drill 0.35) (layers "F.Cu" "B.Cu") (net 1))
 (via (at 113.255093 74.156143) (size 2) (drill 1.2) (layers "F.Cu" "B.Cu") (free yes) (tenting none) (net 1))
 (via (at 103.942941 95.442541) (size 2) (drill 1.2) (layers "F.Cu" "B.Cu") (free yes) (tenting none) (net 1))
 (via (at 115.022859 80.873658) (size 0.8) (drill 0.35) (layers "F.Cu" "B.Cu") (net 1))
 (via (at 97.225427 93.674774) (size 0.8) (drill 0.35) (layers "F.Cu" "B.Cu") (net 1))
 (via (at 119.972607 75.92391) (size 0.8) (drill 0.35) (layers "F.Cu" "B.Cu") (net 1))
 (segment (start 117.497733 78.398783) (end 117.497733 78.398784) (width 0.2) (layer "B.Cu") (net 1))
 (segment (start 113.255093 74.156143) (end 117.497733 78.398783) (width 2) (layer "B.Cu") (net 1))
 (segment (start 103.942941 95.442541) (end 99.700301 91.199901) (width 2) (layer "B.Cu") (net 1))
 (segment (start 99.700301 91.199901) (end 99.700301 91.1999) (width 0.2) (layer "B.Cu") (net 1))
 (segment (start 117.997933 89.698684) (end 117.997933 90.698684) (width 0.4) (layer "F.Cu") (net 4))
 (segment (start 118.552933 89.326184) (end 118.370433 89.326184) (width 0.4) (layer "F.Cu") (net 4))
 (segment (start 99.200101 77.9) (end 99.200101 78.9) (width 0.4) (layer "F.Cu") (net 4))
 (segment (start 100.200101 80.15) (end 100.200101 78.9) (width 0.4) (layer "F.Cu") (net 4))
 (segment (start 118.747933 89.448684) (end 116.997933 89.448684) (width 0.4) (layer "F.Cu") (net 4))
 (segment (start 118.370433 89.326184) (end 117.997933 89.698684) (width 0.4) (layer "F.Cu") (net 4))
 (segment (start 116.997933 89.448684) (end 116.997933 90.698684) (width 0.4) (layer "F.Cu") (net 4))
 (segment (start 100.200101 77.9) (end 99.200101 77.9) (width 0.4) (layer "F.Cu") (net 4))
 (segment (start 98.827601 80.2725) (end 99.200101 79.9) (width 0.4) (layer "F.Cu") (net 4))
 (segment (start 98.645101 80.2725) (end 98.827601 80.2725) (width 0.4) (layer "F.Cu") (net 4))
 (segment (start 118.997933 89.698684) (end 118.747933 89.448684) (width 0.4) (layer "F.Cu") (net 4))
 (segment (start 99.200101 79.9) (end 99.200101 78.9) (width 0.4) (layer "F.Cu") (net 4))
 (segment (start 98.200101 79.9) (end 98.450101 80.15) (width 0.4) (layer "F.Cu") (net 4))
 (segment (start 98.450101 80.15) (end 100.200101 80.15) (width 0.4) (layer "F.Cu") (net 4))
 (segment (start 116.997933 91.698684) (end 117.997933 91.698684) (width 0.4) (layer "F.Cu") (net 4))
 (segment (start 117.997933 90.698684) (end 116.997933 90.698684) (width 0.4) (layer "F.Cu") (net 4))
 (segment (start 100.200101 78.9) (end 100.200101 77.9) (width 0.4) (layer "F.Cu") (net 4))
 (segment (start 116.997933 90.698684) (end 116.997933 91.698684) (width 0.4) (layer "F.Cu") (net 4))
 (segment (start 117.997933 91.698684) (end 117.997933 90.698684) (width 0.4) (layer "F.Cu") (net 4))
 (segment (start 99.200101 78.9) (end 100.200101 78.9) (width 0.4) (layer "F.Cu") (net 4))
 (via (at 100.200101 78.9) (size 0.8) (drill 0.35) (layers "F.Cu" "B.Cu") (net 4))
 (via (at 117.997933 90.698684) (size 0.8) (drill 0.35) (layers "F.Cu" "B.Cu") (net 4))
 (via (at 100.200101 77.9) (size 0.8) (drill 0.35) (layers "F.Cu" "B.Cu") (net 4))
 (via (at 99.200101 77.9) (size 0.8) (drill 0.35) (layers "F.Cu" "B.Cu") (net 4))
 (via (at 116.997933 90.698684) (size 0.8) (drill 0.35) (layers "F.Cu" "B.Cu") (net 4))
 (via (at 116.997933 91.698684) (size 0.8) (drill 0.35) (layers "F.Cu" "B.Cu") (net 4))
 (via (at 117.997933 91.698684) (size 0.8) (drill 0.35) (layers "F.Cu" "B.Cu") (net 4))
 (via (at 99.200101 78.9) (size 0.8) (drill 0.35) (layers "F.Cu" "B.Cu") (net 4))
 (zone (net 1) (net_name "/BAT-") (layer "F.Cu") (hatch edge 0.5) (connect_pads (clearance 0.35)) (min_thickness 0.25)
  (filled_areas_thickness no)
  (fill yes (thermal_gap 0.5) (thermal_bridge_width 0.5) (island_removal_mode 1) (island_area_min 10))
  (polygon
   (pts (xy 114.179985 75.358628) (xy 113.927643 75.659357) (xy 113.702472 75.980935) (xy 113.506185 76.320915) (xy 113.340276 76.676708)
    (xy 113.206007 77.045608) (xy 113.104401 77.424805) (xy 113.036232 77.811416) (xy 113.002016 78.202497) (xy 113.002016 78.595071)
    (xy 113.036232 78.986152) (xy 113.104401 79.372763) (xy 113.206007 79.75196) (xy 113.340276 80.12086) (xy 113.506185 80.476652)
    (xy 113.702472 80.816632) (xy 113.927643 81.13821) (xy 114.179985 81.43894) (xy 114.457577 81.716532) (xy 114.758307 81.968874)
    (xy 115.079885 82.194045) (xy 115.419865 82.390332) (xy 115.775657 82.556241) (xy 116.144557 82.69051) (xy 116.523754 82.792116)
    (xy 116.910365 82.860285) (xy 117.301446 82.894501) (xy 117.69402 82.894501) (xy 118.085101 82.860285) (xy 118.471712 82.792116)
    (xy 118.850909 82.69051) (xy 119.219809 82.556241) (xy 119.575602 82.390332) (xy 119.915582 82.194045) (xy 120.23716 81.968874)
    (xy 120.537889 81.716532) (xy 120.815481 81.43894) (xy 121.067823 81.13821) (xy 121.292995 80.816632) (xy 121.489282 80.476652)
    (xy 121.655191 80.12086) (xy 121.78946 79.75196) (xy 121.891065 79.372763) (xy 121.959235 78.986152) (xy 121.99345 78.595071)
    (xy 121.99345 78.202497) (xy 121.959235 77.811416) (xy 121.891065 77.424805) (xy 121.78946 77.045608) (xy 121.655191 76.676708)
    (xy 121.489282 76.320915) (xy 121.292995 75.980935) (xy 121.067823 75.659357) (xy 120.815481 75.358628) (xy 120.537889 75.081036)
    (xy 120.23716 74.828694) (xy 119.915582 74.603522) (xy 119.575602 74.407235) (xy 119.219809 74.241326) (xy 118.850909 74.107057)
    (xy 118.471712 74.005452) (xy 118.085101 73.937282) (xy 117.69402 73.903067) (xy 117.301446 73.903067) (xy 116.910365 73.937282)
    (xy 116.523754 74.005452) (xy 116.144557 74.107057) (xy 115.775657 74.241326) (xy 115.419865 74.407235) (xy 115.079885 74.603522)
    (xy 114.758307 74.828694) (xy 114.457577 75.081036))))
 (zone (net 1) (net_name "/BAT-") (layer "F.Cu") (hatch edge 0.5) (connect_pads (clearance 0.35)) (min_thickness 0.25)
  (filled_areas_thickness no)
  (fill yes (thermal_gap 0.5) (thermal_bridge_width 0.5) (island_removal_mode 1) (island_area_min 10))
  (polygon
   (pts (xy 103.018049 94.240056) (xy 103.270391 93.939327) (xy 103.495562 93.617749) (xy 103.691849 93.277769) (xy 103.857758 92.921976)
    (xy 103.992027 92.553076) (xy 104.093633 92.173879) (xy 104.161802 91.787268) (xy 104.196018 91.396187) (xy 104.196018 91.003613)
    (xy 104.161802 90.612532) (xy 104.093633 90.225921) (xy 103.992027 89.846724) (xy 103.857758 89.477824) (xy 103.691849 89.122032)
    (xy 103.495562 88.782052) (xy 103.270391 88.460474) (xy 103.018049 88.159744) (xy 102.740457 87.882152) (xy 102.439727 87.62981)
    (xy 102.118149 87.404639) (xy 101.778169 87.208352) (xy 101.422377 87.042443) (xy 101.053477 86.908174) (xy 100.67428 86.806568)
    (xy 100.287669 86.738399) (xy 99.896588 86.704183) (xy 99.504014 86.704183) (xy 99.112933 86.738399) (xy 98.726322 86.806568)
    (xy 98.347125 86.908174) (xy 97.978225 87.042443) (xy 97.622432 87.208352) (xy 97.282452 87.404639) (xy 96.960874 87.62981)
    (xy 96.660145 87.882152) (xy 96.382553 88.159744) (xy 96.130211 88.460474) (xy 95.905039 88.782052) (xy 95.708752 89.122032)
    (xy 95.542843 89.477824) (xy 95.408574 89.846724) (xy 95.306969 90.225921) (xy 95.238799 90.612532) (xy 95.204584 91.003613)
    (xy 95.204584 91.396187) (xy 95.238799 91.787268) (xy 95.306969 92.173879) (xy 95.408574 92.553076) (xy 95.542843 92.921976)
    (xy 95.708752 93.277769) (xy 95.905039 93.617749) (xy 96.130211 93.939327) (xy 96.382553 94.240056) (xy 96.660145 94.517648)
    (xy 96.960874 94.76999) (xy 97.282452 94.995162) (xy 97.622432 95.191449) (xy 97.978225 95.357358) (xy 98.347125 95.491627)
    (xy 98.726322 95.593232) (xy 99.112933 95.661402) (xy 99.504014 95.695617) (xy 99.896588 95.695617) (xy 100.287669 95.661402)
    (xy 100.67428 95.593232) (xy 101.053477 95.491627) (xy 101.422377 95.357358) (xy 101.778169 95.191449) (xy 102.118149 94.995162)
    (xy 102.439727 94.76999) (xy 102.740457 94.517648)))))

